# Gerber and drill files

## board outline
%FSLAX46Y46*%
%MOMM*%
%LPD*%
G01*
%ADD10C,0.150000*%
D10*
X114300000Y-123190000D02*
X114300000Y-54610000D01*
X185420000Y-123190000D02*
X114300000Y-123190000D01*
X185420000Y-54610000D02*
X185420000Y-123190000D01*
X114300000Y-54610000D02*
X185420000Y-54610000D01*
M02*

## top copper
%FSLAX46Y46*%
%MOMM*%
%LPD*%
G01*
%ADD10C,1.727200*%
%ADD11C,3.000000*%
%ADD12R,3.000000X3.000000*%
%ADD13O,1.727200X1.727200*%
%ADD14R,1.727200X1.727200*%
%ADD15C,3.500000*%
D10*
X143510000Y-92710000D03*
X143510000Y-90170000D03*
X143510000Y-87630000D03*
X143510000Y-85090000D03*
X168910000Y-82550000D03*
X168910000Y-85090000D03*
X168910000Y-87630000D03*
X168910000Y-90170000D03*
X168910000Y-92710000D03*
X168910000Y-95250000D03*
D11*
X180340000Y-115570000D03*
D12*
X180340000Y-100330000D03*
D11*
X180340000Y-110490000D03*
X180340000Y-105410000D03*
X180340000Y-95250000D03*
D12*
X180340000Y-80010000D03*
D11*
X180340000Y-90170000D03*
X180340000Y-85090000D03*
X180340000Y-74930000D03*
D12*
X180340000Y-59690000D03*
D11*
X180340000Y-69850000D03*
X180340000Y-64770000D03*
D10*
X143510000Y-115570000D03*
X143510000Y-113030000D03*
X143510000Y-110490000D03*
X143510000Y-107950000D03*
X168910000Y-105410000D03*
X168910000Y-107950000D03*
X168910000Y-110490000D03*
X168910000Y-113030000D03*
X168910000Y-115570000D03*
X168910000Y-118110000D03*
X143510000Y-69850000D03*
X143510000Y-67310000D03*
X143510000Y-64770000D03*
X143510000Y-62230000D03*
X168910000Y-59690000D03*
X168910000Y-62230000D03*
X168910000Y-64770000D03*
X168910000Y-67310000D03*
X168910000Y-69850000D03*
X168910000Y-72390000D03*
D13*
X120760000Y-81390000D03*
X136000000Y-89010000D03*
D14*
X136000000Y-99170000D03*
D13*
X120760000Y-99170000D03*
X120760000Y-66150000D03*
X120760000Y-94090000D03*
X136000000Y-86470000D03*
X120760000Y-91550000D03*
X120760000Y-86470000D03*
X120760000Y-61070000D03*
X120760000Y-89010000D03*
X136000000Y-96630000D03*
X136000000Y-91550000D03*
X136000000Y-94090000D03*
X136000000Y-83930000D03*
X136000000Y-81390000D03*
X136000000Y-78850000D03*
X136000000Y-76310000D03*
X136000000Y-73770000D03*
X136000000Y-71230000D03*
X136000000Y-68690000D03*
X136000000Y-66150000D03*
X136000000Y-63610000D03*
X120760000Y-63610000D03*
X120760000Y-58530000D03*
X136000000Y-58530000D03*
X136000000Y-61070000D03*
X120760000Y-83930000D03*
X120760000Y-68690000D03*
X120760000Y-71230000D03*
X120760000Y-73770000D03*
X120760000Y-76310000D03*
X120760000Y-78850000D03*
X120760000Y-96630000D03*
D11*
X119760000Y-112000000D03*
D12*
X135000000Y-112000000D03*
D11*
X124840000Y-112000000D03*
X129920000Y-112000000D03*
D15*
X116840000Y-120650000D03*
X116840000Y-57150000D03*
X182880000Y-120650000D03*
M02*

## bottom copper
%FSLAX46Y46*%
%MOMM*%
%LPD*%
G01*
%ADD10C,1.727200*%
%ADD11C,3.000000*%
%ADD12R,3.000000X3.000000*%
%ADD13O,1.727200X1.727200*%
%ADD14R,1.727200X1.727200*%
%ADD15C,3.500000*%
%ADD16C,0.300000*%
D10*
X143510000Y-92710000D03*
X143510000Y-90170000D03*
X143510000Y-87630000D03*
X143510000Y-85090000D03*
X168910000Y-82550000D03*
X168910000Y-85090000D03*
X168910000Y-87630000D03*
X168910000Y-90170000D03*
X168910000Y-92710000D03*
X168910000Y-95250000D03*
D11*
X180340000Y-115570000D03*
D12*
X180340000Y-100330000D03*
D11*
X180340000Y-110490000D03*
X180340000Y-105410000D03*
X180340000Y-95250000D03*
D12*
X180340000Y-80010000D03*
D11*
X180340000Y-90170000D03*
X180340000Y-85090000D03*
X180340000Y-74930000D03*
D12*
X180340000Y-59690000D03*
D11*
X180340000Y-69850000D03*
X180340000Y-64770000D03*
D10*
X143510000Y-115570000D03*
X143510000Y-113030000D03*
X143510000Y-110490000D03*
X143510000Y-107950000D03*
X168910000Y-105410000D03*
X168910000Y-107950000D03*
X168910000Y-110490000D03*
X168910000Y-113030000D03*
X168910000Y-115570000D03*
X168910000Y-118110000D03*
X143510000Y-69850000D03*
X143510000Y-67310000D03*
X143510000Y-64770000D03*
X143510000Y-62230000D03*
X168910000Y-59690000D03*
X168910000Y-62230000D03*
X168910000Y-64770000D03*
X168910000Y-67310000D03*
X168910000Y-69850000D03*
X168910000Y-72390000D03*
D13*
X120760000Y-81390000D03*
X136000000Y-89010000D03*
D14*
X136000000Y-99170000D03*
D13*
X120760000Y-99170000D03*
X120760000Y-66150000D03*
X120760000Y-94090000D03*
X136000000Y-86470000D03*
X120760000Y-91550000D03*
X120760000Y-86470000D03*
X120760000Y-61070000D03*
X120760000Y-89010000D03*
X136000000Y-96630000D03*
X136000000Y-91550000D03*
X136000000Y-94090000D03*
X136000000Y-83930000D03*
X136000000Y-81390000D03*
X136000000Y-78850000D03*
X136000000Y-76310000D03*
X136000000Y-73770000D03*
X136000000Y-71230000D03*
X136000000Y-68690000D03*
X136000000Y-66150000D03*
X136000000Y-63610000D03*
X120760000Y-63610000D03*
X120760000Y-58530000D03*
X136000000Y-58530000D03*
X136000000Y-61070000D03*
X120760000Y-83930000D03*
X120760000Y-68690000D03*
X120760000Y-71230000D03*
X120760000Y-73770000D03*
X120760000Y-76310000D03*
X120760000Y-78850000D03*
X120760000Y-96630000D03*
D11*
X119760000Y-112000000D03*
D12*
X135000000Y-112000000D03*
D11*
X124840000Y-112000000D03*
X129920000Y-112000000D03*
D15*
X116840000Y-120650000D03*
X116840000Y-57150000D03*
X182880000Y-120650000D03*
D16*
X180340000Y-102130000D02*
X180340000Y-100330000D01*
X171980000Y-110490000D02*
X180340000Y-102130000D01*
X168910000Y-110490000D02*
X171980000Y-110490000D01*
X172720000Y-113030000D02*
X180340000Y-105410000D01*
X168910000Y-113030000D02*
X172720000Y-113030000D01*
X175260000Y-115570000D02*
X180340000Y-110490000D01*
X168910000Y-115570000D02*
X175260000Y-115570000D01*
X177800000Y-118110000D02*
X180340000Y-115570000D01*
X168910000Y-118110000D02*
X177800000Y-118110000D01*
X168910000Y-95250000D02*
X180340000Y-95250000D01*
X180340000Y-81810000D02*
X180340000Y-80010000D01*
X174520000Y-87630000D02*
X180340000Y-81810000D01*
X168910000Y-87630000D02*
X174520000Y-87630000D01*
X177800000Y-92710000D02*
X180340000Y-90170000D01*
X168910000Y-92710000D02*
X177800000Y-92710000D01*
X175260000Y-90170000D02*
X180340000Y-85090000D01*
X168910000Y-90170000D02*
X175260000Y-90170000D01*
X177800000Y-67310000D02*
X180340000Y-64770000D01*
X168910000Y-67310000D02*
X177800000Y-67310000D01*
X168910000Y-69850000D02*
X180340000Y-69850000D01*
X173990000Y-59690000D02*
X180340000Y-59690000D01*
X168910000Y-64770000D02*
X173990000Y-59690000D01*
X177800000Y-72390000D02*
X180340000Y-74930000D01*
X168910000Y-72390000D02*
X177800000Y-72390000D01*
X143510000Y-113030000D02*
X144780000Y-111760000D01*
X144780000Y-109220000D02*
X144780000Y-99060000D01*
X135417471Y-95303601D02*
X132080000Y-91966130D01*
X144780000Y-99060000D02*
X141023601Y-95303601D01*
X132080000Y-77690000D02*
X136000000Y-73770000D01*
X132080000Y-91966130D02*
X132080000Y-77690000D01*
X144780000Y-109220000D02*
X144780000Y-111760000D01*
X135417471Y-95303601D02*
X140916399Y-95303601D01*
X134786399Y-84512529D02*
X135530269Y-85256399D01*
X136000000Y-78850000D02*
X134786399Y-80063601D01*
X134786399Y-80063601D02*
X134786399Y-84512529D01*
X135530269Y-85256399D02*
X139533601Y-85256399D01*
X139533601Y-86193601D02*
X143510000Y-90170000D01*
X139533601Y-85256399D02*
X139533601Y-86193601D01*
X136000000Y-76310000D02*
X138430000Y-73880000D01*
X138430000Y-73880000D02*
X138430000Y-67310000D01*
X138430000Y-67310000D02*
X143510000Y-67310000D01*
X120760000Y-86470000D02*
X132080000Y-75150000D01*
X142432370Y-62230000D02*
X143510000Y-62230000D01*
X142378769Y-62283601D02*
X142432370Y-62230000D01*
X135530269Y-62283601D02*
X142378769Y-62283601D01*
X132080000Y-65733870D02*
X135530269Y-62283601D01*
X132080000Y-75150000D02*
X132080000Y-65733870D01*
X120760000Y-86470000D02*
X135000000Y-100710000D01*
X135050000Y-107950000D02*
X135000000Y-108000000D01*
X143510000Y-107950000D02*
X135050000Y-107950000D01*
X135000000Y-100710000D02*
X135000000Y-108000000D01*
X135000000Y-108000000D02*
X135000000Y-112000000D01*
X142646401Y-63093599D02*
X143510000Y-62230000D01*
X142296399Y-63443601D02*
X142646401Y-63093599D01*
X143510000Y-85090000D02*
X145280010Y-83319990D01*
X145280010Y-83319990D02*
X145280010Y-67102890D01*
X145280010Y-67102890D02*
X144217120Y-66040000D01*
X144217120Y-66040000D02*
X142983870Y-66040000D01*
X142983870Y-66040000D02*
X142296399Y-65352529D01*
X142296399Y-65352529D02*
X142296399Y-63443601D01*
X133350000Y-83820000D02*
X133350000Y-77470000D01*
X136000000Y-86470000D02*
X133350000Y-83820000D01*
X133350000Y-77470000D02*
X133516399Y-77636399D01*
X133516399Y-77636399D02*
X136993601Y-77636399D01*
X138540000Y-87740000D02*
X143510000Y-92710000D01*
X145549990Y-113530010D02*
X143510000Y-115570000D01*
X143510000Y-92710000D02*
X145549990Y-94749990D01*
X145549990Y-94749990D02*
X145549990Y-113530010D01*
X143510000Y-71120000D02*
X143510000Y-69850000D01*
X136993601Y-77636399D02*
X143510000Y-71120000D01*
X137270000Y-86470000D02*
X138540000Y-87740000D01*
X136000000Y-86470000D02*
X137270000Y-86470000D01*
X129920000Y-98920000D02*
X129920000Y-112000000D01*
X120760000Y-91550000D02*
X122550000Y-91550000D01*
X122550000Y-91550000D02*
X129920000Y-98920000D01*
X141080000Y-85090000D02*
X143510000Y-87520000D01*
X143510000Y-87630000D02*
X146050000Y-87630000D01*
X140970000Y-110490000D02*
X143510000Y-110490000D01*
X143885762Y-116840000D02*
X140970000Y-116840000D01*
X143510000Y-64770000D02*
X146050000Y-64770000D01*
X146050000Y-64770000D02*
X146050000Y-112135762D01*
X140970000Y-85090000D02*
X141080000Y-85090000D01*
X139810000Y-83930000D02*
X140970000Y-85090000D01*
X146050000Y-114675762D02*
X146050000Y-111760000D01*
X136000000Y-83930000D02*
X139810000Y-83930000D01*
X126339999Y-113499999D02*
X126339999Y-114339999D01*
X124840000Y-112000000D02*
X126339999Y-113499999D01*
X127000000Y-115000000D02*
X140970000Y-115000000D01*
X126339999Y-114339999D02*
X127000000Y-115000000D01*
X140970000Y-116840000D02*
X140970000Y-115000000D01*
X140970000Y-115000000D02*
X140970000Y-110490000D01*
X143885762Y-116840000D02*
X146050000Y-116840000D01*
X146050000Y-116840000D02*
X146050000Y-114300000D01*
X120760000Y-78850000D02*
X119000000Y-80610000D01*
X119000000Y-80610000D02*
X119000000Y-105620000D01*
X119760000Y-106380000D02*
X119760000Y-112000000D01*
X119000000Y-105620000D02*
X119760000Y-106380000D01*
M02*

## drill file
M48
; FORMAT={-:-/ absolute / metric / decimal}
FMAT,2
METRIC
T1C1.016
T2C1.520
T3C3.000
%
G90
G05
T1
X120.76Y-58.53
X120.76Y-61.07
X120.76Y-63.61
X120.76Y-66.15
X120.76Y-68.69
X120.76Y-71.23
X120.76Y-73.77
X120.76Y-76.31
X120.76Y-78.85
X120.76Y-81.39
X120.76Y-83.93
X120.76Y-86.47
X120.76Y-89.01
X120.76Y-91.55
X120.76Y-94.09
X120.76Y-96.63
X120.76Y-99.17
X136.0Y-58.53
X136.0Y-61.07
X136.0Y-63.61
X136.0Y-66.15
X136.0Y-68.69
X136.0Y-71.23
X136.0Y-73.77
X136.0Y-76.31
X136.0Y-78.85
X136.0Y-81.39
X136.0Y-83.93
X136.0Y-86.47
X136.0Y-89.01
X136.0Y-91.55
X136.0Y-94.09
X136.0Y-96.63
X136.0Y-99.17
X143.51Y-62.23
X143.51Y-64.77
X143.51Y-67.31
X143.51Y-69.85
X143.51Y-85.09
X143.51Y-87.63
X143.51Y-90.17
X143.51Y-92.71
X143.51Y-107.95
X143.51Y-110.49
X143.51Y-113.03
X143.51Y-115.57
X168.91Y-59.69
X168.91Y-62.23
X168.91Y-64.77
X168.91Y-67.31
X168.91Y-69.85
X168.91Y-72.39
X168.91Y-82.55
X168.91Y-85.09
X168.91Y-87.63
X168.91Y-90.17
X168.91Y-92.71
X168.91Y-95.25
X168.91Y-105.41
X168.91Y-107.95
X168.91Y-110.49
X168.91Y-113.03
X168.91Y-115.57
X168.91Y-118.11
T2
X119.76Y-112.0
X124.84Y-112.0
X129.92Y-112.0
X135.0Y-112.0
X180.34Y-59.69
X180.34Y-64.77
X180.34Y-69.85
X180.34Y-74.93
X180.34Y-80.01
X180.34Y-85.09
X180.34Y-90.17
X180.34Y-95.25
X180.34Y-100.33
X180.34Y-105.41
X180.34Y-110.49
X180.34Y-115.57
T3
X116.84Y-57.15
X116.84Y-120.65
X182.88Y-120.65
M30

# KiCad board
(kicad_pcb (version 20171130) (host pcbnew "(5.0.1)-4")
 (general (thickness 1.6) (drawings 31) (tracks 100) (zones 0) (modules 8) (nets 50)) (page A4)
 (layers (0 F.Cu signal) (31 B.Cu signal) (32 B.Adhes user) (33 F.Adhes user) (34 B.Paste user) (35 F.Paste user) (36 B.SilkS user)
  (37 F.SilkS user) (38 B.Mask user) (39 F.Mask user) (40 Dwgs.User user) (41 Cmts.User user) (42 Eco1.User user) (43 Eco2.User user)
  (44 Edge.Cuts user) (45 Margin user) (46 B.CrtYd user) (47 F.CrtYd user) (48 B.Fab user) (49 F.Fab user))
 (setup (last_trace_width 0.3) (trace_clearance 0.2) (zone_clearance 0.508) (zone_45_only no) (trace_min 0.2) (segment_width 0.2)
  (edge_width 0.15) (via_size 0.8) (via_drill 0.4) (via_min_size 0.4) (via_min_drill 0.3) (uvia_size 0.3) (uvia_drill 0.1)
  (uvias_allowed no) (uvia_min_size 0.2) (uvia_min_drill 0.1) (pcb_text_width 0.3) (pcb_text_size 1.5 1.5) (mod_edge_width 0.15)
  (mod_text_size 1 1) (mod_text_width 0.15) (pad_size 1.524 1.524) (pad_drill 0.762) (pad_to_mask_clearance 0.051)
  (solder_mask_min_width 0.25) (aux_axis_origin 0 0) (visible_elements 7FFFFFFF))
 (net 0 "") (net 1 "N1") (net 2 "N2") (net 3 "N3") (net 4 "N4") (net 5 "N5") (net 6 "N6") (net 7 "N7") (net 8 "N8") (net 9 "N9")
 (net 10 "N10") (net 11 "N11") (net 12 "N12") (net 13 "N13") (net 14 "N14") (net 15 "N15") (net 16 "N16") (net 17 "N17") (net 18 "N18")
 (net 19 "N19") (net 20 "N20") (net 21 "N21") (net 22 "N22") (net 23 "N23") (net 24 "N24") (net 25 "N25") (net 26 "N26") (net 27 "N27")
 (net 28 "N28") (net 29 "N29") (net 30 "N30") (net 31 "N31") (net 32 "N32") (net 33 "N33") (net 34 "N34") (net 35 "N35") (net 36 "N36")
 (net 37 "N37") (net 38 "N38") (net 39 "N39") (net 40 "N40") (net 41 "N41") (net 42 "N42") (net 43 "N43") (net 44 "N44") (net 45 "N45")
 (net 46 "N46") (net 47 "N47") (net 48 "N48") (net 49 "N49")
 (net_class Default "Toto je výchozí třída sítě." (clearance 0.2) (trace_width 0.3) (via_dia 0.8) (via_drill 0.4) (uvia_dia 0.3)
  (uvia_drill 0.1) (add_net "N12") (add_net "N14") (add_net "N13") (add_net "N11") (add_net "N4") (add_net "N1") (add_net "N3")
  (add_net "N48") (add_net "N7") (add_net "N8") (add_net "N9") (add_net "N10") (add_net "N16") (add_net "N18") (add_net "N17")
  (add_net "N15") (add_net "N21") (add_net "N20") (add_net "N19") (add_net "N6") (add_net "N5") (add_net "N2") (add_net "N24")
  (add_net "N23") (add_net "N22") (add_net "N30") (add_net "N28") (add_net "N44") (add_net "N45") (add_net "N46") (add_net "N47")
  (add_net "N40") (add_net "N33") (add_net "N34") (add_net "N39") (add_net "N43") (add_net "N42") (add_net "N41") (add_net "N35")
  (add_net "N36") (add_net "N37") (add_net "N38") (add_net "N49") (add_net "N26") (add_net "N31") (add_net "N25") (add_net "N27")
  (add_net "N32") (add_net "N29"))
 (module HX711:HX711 (layer F.Cu) (at 167.64 91.44 180)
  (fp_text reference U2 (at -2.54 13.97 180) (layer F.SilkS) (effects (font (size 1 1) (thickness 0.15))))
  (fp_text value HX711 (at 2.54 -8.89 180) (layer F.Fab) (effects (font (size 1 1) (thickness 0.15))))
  (pad 7 thru_hole circle (at 24.13 -1.27 180) (size 1.7272 1.7272) (drill 1.016) (layers *.Cu *.Mask) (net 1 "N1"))
  (pad 8 thru_hole circle (at 24.13 1.27 180) (size 1.7272 1.7272) (drill 1.016) (layers *.Cu *.Mask) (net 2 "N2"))
  (pad 9 thru_hole circle (at 24.13 3.81 180) (size 1.7272 1.7272) (drill 1.016) (layers *.Cu *.Mask) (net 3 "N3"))
  (pad 10 thru_hole circle (at 24.13 6.35 180) (size 1.7272 1.7272) (drill 1.016) (layers *.Cu *.Mask) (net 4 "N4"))
  (pad 6 thru_hole circle (at -1.27 8.89 180) (size 1.7272 1.7272) (drill 1.016) (layers *.Cu *.Mask) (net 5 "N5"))
  (pad 5 thru_hole circle (at -1.27 6.35 180) (size 1.7272 1.7272) (drill 1.016) (layers *.Cu *.Mask) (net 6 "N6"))
  (pad 4 thru_hole circle (at -1.27 3.81 180) (size 1.7272 1.7272) (drill 1.016) (layers *.Cu *.Mask) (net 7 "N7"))
  (pad 3 thru_hole circle (at -1.27 1.27 180) (size 1.7272 1.7272) (drill 1.016) (layers *.Cu *.Mask) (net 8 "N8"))
  (pad 2 thru_hole circle (at -1.27 -1.27 180) (size 1.7272 1.7272) (drill 1.016) (layers *.Cu *.Mask) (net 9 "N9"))
  (pad 1 thru_hole circle (at -1.27 -3.81 180) (size 1.7272 1.7272) (drill 1.016) (layers *.Cu *.Mask) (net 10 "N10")))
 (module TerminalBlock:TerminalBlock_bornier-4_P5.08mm (layer F.Cu) (at 180.34 100.33 270)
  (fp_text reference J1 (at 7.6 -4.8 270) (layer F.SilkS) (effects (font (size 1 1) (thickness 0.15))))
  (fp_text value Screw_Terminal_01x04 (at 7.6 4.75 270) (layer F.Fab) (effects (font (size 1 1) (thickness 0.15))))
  (pad 4 thru_hole circle (at 15.24 0 270) (size 3 3) (drill 1.52) (layers *.Cu *.Mask) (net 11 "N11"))
  (pad 1 thru_hole rect (at 0 0 270) (size 3 3) (drill 1.52) (layers *.Cu *.Mask) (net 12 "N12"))
  (pad 3 thru_hole circle (at 10.16 0 270) (size 3 3) (drill 1.52) (layers *.Cu *.Mask) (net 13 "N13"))
  (pad 2 thru_hole circle (at 5.08 0 270) (size 3 3) (drill 1.52) (layers *.Cu *.Mask) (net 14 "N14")))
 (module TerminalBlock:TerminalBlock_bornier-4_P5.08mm (layer F.Cu) (at 180.34 80.01 270)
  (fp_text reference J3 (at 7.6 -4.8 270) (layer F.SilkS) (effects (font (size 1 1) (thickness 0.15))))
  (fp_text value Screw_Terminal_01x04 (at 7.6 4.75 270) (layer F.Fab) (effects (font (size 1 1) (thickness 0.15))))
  (pad 4 thru_hole circle (at 15.24 0 270) (size 3 3) (drill 1.52) (layers *.Cu *.Mask) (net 10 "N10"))
  (pad 1 thru_hole rect (at 0 0 270) (size 3 3) (drill 1.52) (layers *.Cu *.Mask) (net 7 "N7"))
  (pad 3 thru_hole circle (at 10.16 0 270) (size 3 3) (drill 1.52) (layers *.Cu *.Mask) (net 9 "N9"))
  (pad 2 thru_hole circle (at 5.08 0 270) (size 3 3) (drill 1.52) (layers *.Cu *.Mask) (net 8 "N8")))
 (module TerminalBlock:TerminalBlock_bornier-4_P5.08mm (layer F.Cu) (at 180.34 59.69 270)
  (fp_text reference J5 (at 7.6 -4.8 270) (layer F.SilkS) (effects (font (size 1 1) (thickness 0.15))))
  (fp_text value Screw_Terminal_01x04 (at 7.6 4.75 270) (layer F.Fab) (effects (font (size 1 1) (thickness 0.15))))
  (pad 4 thru_hole circle (at 15.24 0 270) (size 3 3) (drill 1.52) (layers *.Cu *.Mask) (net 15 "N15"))
  (pad 1 thru_hole rect (at 0 0 270) (size 3 3) (drill 1.52) (layers *.Cu *.Mask) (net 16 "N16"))
  (pad 3 thru_hole circle (at 10.16 0 270) (size 3 3) (drill 1.52) (layers *.Cu *.Mask) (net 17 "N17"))
  (pad 2 thru_hole circle (at 5.08 0 270) (size 3 3) (drill 1.52) (layers *.Cu *.Mask) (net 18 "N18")))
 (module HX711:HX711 (layer F.Cu) (at 167.64 114.3 180)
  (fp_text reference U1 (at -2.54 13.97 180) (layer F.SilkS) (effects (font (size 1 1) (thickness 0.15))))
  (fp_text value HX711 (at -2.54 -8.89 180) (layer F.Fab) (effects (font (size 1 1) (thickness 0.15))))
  (pad 7 thru_hole circle (at 24.13 -1.27 180) (size 1.7272 1.7272) (drill 1.016) (layers *.Cu *.Mask) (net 1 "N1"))
  (pad 8 thru_hole circle (at 24.13 1.27 180) (size 1.7272 1.7272) (drill 1.016) (layers *.Cu *.Mask) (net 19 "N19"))
  (pad 9 thru_hole circle (at 24.13 3.81 180) (size 1.7272 1.7272) (drill 1.016) (layers *.Cu *.Mask) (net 3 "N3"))
  (pad 10 thru_hole circle (at 24.13 6.35 180) (size 1.7272 1.7272) (drill 1.016) (layers *.Cu *.Mask) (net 4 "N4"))
  (pad 6 thru_hole circle (at -1.27 8.89 180) (size 1.7272 1.7272) (drill 1.016) (layers *.Cu *.Mask) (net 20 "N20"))
  (pad 5 thru_hole circle (at -1.27 6.35 180) (size 1.7272 1.7272) (drill 1.016) (layers *.Cu *.Mask) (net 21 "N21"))
  (pad 4 thru_hole circle (at -1.27 3.81 180) (size 1.7272 1.7272) (drill 1.016) (layers *.Cu *.Mask) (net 12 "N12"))
  (pad 3 thru_hole circle (at -1.27 1.27 180) (size 1.7272 1.7272) (drill 1.016) (layers *.Cu *.Mask) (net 14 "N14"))
  (pad 2 thru_hole circle (at -1.27 -1.27 180) (size 1.7272 1.7272) (drill 1.016) (layers *.Cu *.Mask) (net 13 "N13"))
  (pad 1 thru_hole circle (at -1.27 -3.81 180) (size 1.7272 1.7272) (drill 1.016) (layers *.Cu *.Mask) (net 11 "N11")))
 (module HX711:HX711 (layer F.Cu) (at 167.64 68.58 180)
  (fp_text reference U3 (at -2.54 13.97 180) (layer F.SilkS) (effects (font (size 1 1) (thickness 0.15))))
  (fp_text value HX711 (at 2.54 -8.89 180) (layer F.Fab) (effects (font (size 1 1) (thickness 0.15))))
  (pad 7 thru_hole circle (at 24.13 -1.27 180) (size 1.7272 1.7272) (drill 1.016) (layers *.Cu *.Mask) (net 1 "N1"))
  (pad 8 thru_hole circle (at 24.13 1.27 180) (size 1.7272 1.7272) (drill 1.016) (layers *.Cu *.Mask) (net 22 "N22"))
  (pad 9 thru_hole circle (at 24.13 3.81 180) (size 1.7272 1.7272) (drill 1.016) (layers *.Cu *.Mask) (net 3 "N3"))
  (pad 10 thru_hole circle (at 24.13 6.35 180) (size 1.7272 1.7272) (drill 1.016) (layers *.Cu *.Mask) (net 4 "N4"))
  (pad 6 thru_hole circle (at -1.27 8.89 180) (size 1.7272 1.7272) (drill 1.016) (layers *.Cu *.Mask) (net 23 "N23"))
  (pad 5 thru_hole circle (at -1.27 6.35 180) (size 1.7272 1.7272) (drill 1.016) (layers *.Cu *.Mask) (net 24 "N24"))
  (pad 4 thru_hole circle (at -1.27 3.81 180) (size 1.7272 1.7272) (drill 1.016) (layers *.Cu *.Mask) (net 16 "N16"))
  (pad 3 thru_hole circle (at -1.27 1.27 180) (size 1.7272 1.7272) (drill 1.016) (layers *.Cu *.Mask) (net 18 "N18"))
  (pad 2 thru_hole circle (at -1.27 -1.27 180) (size 1.7272 1.7272) (drill 1.016) (layers *.Cu *.Mask) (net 17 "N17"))
  (pad 1 thru_hole circle (at -1.27 -3.81 180) (size 1.7272 1.7272) (drill 1.016) (layers *.Cu *.Mask) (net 15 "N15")))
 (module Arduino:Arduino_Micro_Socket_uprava (layer F.Cu) (at 119.38 54.61 270)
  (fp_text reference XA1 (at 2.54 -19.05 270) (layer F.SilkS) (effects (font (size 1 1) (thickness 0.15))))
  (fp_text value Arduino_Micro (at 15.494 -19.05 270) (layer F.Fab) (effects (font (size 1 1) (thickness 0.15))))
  (pad "" thru_hole oval (at 26.78 -1.38 270) (size 1.7272 1.7272) (drill 1.016) (layers *.Cu *.Mask))
  (pad RST2 thru_hole oval (at 34.4 -16.62 270) (size 1.7272 1.7272) (drill 1.016) (layers *.Cu *.Mask) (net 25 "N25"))
  (pad MOSI thru_hole rect (at 44.56 -16.62 270) (size 1.7272 1.7272) (drill 1.016) (layers *.Cu *.Mask) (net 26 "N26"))
  (pad SCK thru_hole oval (at 44.56 -1.38 270) (size 1.7272 1.7272) (drill 1.016) (layers *.Cu *.Mask) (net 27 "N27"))
  (pad A0 thru_hole oval (at 11.54 -1.38 270) (size 1.7272 1.7272) (drill 1.016) (layers *.Cu *.Mask) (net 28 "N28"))
  (pad VIN thru_hole oval (at 39.48 -1.38 270) (size 1.7272 1.7272) (drill 1.016) (layers *.Cu *.Mask) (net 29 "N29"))
  (pad GND2 thru_hole oval (at 31.86 -16.62 270) (size 1.7272 1.7272) (drill 1.016) (layers *.Cu *.Mask) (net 1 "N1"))
  (pad GND1 thru_hole oval (at 36.94 -1.38 270) (size 1.7272 1.7272) (drill 1.016) (layers *.Cu *.Mask) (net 1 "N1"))
  (pad 5V thru_hole oval (at 31.86 -1.38 270) (size 1.7272 1.7272) (drill 1.016) (layers *.Cu *.Mask) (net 4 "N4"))
  (pad 3V3 thru_hole oval (at 6.46 -1.38 270) (size 1.7272 1.7272) (drill 1.016) (layers *.Cu *.Mask) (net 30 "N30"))
  (pad RST1 thru_hole oval (at 34.4 -1.38 270) (size 1.7272 1.7272) (drill 1.016) (layers *.Cu *.Mask) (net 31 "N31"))
  (pad SS thru_hole oval (at 42.02 -16.62 270) (size 1.7272 1.7272) (drill 1.016) (layers *.Cu *.Mask) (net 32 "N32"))
  (pad D0 thru_hole oval (at 36.94 -16.62 270) (size 1.7272 1.7272) (drill 1.016) (layers *.Cu *.Mask) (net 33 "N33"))
  (pad D1 thru_hole oval (at 39.48 -16.62 270) (size 1.7272 1.7272) (drill 1.016) (layers *.Cu *.Mask) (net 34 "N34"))
  (pad D2 thru_hole oval (at 29.32 -16.62 270) (size 1.7272 1.7272) (drill 1.016) (layers *.Cu *.Mask) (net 3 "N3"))
  (pad D3 thru_hole oval (at 26.78 -16.62 270) (size 1.7272 1.7272) (drill 1.016) (layers *.Cu *.Mask) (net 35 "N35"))
  (pad D4 thru_hole oval (at 24.24 -16.62 270) (size 1.7272 1.7272) (drill 1.016) (layers *.Cu *.Mask) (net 2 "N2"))
  (pad D5 thru_hole oval (at 21.7 -16.62 270) (size 1.7272 1.7272) (drill 1.016) (layers *.Cu *.Mask) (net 22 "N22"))
  (pad D6 thru_hole oval (at 19.16 -16.62 270) (size 1.7272 1.7272) (drill 1.016) (layers *.Cu *.Mask) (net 19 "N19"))
  (pad D7 thru_hole oval (at 16.62 -16.62 270) (size 1.7272 1.7272) (drill 1.016) (layers *.Cu *.Mask) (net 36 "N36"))
  (pad D8 thru_hole oval (at 14.08 -16.62 270) (size 1.7272 1.7272) (drill 1.016) (layers *.Cu *.Mask) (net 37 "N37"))
  (pad D9 thru_hole oval (at 11.54 -16.62 270) (size 1.7272 1.7272) (drill 1.016) (layers *.Cu *.Mask) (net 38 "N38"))
  (pad D10 thru_hole oval (at 9 -16.62 270) (size 1.7272 1.7272) (drill 1.016) (layers *.Cu *.Mask) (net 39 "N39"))
  (pad AREF thru_hole oval (at 9 -1.38 270) (size 1.7272 1.7272) (drill 1.016) (layers *.Cu *.Mask) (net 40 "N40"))
  (pad D13 thru_hole oval (at 3.92 -1.38 270) (size 1.7272 1.7272) (drill 1.016) (layers *.Cu *.Mask) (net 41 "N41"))
  (pad D12 thru_hole oval (at 3.92 -16.62 270) (size 1.7272 1.7272) (drill 1.016) (layers *.Cu *.Mask) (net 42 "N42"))
  (pad D11 thru_hole oval (at 6.46 -16.62 270) (size 1.7272 1.7272) (drill 1.016) (layers *.Cu *.Mask) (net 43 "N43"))
  (pad "" thru_hole oval (at 29.32 -1.38 270) (size 1.7272 1.7272) (drill 1.016) (layers *.Cu *.Mask))
  (pad A1 thru_hole oval (at 14.08 -1.38 270) (size 1.7272 1.7272) (drill 1.016) (layers *.Cu *.Mask) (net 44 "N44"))
  (pad A2 thru_hole oval (at 16.62 -1.38 270) (size 1.7272 1.7272) (drill 1.016) (layers *.Cu *.Mask) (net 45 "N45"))
  (pad A3 thru_hole oval (at 19.16 -1.38 270) (size 1.7272 1.7272) (drill 1.016) (layers *.Cu *.Mask) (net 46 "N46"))
  (pad A4 thru_hole oval (at 21.7 -1.38 270) (size 1.7272 1.7272) (drill 1.016) (layers *.Cu *.Mask) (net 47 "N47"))
  (pad A5 thru_hole oval (at 24.24 -1.38 270) (size 1.7272 1.7272) (drill 1.016) (layers *.Cu *.Mask) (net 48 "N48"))
  (pad MISO thru_hole oval (at 42.02 -1.38 270) (size 1.7272 1.7272) (drill 1.016) (layers *.Cu *.Mask) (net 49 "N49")))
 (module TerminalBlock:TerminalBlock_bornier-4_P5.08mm (layer F.Cu) (at 135 112 180)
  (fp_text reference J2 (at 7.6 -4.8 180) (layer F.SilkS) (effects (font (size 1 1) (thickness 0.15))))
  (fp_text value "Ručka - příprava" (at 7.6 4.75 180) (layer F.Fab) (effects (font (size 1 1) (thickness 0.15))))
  (pad 4 thru_hole circle (at 15.24 0 180) (size 3 3) (drill 1.52) (layers *.Cu *.Mask) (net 48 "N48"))
  (pad 1 thru_hole rect (at 0 0 180) (size 3 3) (drill 1.52) (layers *.Cu *.Mask) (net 4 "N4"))
  (pad 3 thru_hole circle (at 10.16 0 180) (size 3 3) (drill 1.52) (layers *.Cu *.Mask) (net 3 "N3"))
  (pad 2 thru_hole circle (at 5.08 0 180) (size 3 3) (drill 1.52) (layers *.Cu *.Mask) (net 1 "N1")))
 (gr_line (start 114.3 123.19) (end 114.3 54.61) (layer Edge.Cuts) (width 0.15))
 (gr_line (start 185.42 123.19) (end 114.3 123.19) (layer Edge.Cuts) (width 0.15))
 (gr_line (start 185.42 54.61) (end 185.42 123.19) (layer Edge.Cuts) (width 0.15))
 (gr_line (start 114.3 54.61) (end 185.42 54.61) (layer Edge.Cuts) (width 0.15))
 (via (at 116.84 120.65) (size 3.5) (drill 3) (layers F.Cu B.Cu) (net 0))
 (via (at 116.84 57.15) (size 3.5) (drill 3) (layers F.Cu B.Cu) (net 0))
 (via (at 182.88 120.65) (size 3.5) (drill 3) (layers F.Cu B.Cu) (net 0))
 (segment (start 180.34 102.13) (end 180.34 100.33) (width 0.3) (layer B.Cu) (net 12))
 (segment (start 171.98 110.49) (end 180.34 102.13) (width 0.3) (layer B.Cu) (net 12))
 (segment (start 168.91 110.49) (end 171.98 110.49) (width 0.3) (layer B.Cu) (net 12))
 (segment (start 172.72 113.03) (end 180.34 105.41) (width 0.3) (layer B.Cu) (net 14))
 (segment (start 168.91 113.03) (end 172.72 113.03) (width 0.3) (layer B.Cu) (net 14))
 (segment (start 175.26 115.57) (end 180.34 110.49) (width 0.3) (layer B.Cu) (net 13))
 (segment (start 168.91 115.57) (end 175.26 115.57) (width 0.3) (layer B.Cu) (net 13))
 (segment (start 177.8 118.11) (end 180.34 115.57) (width 0.3) (layer B.Cu) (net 11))
 (segment (start 168.91 118.11) (end 177.8 118.11) (width 0.3) (layer B.Cu) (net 11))
 (segment (start 168.91 95.25) (end 180.34 95.25) (width 0.3) (layer B.Cu) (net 10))
 (segment (start 180.34 81.81) (end 180.34 80.01) (width 0.3) (layer B.Cu) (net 7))
 (segment (start 174.52 87.63) (end 180.34 81.81) (width 0.3) (layer B.Cu) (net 7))
 (segment (start 168.91 87.63) (end 174.52 87.63) (width 0.3) (layer B.Cu) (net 7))
 (segment (start 177.8 92.71) (end 180.34 90.17) (width 0.3) (layer B.Cu) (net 9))
 (segment (start 168.91 92.71) (end 177.8 92.71) (width 0.3) (layer B.Cu) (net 9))
 (segment (start 175.26 90.17) (end 180.34 85.09) (width 0.3) (layer B.Cu) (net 8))
 (segment (start 168.91 90.17) (end 175.26 90.17) (width 0.3) (layer B.Cu) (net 8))
 (segment (start 177.8 67.31) (end 180.34 64.77) (width 0.3) (layer B.Cu) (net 18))
 (segment (start 168.91 67.31) (end 177.8 67.31) (width 0.3) (layer B.Cu) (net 18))
 (segment (start 168.91 69.85) (end 180.34 69.85) (width 0.3) (layer B.Cu) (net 17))
 (segment (start 173.99 59.69) (end 180.34 59.69) (width 0.3) (layer B.Cu) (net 16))
 (segment (start 168.91 64.77) (end 173.99 59.69) (width 0.3) (layer B.Cu) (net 16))
 (segment (start 177.8 72.39) (end 180.34 74.93) (width 0.3) (layer B.Cu) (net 15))
 (segment (start 168.91 72.39) (end 177.8 72.39) (width 0.3) (layer B.Cu) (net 15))
 (segment (start 143.51 113.03) (end 144.78 111.76) (width 0.3) (layer B.Cu) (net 19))
 (segment (start 144.78 109.22) (end 144.78 99.06) (width 0.3) (layer B.Cu) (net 19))
 (segment (start 135.417471 95.303601) (end 132.08 91.96613) (width 0.3) (layer B.Cu) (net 19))
 (segment (start 144.78 99.06) (end 141.023601 95.303601) (width 0.3) (layer B.Cu) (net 19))
 (segment (start 132.08 77.69) (end 136 73.77) (width 0.3) (layer B.Cu) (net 19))
 (segment (start 132.08 91.96613) (end 132.08 77.69) (width 0.3) (layer B.Cu) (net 19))
 (segment (start 144.78 109.22) (end 144.78 111.76) (width 0.3) (layer B.Cu) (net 19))
 (segment (start 135.417471 95.303601) (end 140.916399 95.303601) (width 0.3) (layer B.Cu) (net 19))
 (segment (start 134.786399 84.512529) (end 135.530269 85.256399) (width 0.3) (layer B.Cu) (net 2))
 (segment (start 136 78.85) (end 134.786399 80.063601) (width 0.3) (layer B.Cu) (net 2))
 (segment (start 134.786399 80.063601) (end 134.786399 84.512529) (width 0.3) (layer B.Cu) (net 2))
 (segment (start 135.530269 85.256399) (end 139.533601 85.256399) (width 0.3) (layer B.Cu) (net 2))
 (segment (start 139.533601 86.193601) (end 143.51 90.17) (width 0.3) (layer B.Cu) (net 2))
 (segment (start 139.533601 85.256399) (end 139.533601 86.193601) (width 0.3) (layer B.Cu) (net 2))
 (segment (start 136 76.31) (end 138.43 73.88) (width 0.3) (layer B.Cu) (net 22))
 (segment (start 138.43 73.88) (end 138.43 67.31) (width 0.3) (layer B.Cu) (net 22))
 (segment (start 138.43 67.31) (end 143.51 67.31) (width 0.3) (layer B.Cu) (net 22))
 (segment (start 120.76 86.47) (end 132.08 75.15) (width 0.3) (layer B.Cu) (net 4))
 (segment (start 142.43237 62.23) (end 143.51 62.23) (width 0.3) (layer B.Cu) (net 4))
 (segment (start 142.378769 62.283601) (end 142.43237 62.23) (width 0.3) (layer B.Cu) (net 4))
 (segment (start 135.530269 62.283601) (end 142.378769 62.283601) (width 0.3) (layer B.Cu) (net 4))
 (segment (start 132.08 65.73387) (end 135.530269 62.283601) (width 0.3) (layer B.Cu) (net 4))
 (segment (start 132.08 75.15) (end 132.08 65.73387) (width 0.3) (layer B.Cu) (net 4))
 (segment (start 120.76 86.47) (end 135 100.71) (width 0.3) (layer B.Cu) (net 4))
 (segment (start 135.05 107.95) (end 135 108) (width 0.3) (layer B.Cu) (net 4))
 (segment (start 143.51 107.95) (end 135.05 107.95) (width 0.3) (layer B.Cu) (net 4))
 (segment (start 135 100.71) (end 135 108) (width 0.3) (layer B.Cu) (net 4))
 (segment (start 135 108) (end 135 112) (width 0.3) (layer B.Cu) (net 4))
 (segment (start 142.646401 63.093599) (end 143.51 62.23) (width 0.3) (layer B.Cu) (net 4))
 (segment (start 142.296399 63.443601) (end 142.646401 63.093599) (width 0.3) (layer B.Cu) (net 4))
 (segment (start 143.51 85.09) (end 145.28001 83.31999) (width 0.3) (layer B.Cu) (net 4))
 (segment (start 145.28001 83.31999) (end 145.28001 67.10289) (width 0.3) (layer B.Cu) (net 4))
 (segment (start 145.28001 67.10289) (end 144.21712 66.04) (width 0.3) (layer B.Cu) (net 4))
 (segment (start 144.21712 66.04) (end 142.98387 66.04) (width 0.3) (layer B.Cu) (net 4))
 (segment (start 142.98387 66.04) (end 142.296399 65.352529) (width 0.3) (layer B.Cu) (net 4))
 (segment (start 142.296399 65.352529) (end 142.296399 63.443601) (width 0.3) (layer B.Cu) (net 4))
 (segment (start 133.35 83.82) (end 133.35 77.47) (width 0.3) (layer B.Cu) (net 1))
 (segment (start 136 86.47) (end 133.35 83.82) (width 0.3) (layer B.Cu) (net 1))
 (segment (start 133.35 77.47) (end 133.516399 77.636399) (width 0.3) (layer B.Cu) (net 1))
 (segment (start 133.516399 77.636399) (end 136.993601 77.636399) (width 0.3) (layer B.Cu) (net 1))
 (segment (start 138.54 87.74) (end 143.51 92.71) (width 0.3) (layer B.Cu) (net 1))
 (segment (start 145.54999 113.53001) (end 143.51 115.57) (width 0.3) (layer B.Cu) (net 1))
 (segment (start 143.51 92.71) (end 145.54999 94.74999) (width 0.3) (layer B.Cu) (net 1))
 (segment (start 145.54999 94.74999) (end 145.54999 113.53001) (width 0.3) (layer B.Cu) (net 1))
 (segment (start 143.51 71.12) (end 143.51 69.85) (width 0.3) (layer B.Cu) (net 1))
 (segment (start 136.993601 77.636399) (end 143.51 71.12) (width 0.3) (layer B.Cu) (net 1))
 (segment (start 137.27 86.47) (end 138.54 87.74) (width 0.3) (layer B.Cu) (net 1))
 (segment (start 136 86.47) (end 137.27 86.47) (width 0.3) (layer B.Cu) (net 1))
 (segment (start 129.92 98.92) (end 129.92 112) (width 0.3) (layer B.Cu) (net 1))
 (segment (start 120.76 91.55) (end 122.55 91.55) (width 0.3) (layer B.Cu) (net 1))
 (segment (start 122.55 91.55) (end 129.92 98.92) (width 0.3) (layer B.Cu) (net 1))
 (segment (start 141.08 85.09) (end 143.51 87.52) (width 0.3) (layer B.Cu) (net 3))
 (segment (start 143.51 87.63) (end 146.05 87.63) (width 0.3) (layer B.Cu) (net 3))
 (segment (start 140.97 110.49) (end 143.51 110.49) (width 0.3) (layer B.Cu) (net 3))
 (segment (start 143.885762 116.84) (end 140.97 116.84) (width 0.3) (layer B.Cu) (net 3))
 (segment (start 143.51 64.77) (end 146.05 64.77) (width 0.3) (layer B.Cu) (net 3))
 (segment (start 146.05 64.77) (end 146.05 112.135762) (width 0.3) (layer B.Cu) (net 3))
 (segment (start 140.97 85.09) (end 141.08 85.09) (width 0.3) (layer B.Cu) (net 3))
 (segment (start 139.81 83.93) (end 140.97 85.09) (width 0.3) (layer B.Cu) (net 3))
 (segment (start 146.05 114.675762) (end 146.05 111.76) (width 0.3) (layer B.Cu) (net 3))
 (segment (start 136 83.93) (end 139.81 83.93) (width 0.3) (layer B.Cu) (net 3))
 (segment (start 126.339999 113.499999) (end 126.339999 114.339999) (width 0.3) (layer B.Cu) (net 3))
 (segment (start 124.84 112) (end 126.339999 113.499999) (width 0.3) (layer B.Cu) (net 3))
 (segment (start 127 115) (end 140.97 115) (width 0.3) (layer B.Cu) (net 3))
 (segment (start 126.339999 114.339999) (end 127 115) (width 0.3) (layer B.Cu) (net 3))
 (segment (start 140.97 116.84) (end 140.97 115) (width 0.3) (layer B.Cu) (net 3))
 (segment (start 140.97 115) (end 140.97 110.49) (width 0.3) (layer B.Cu) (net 3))
 (segment (start 143.885762 116.84) (end 146.05 116.84) (width 0.3) (layer B.Cu) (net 3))
 (segment (start 146.05 116.84) (end 146.05 114.3) (width 0.3) (layer B.Cu) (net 3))
 (segment (start 120.76 78.85) (end 119 80.61) (width 0.3) (layer B.Cu) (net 48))
 (segment (start 119 80.61) (end 119 105.62) (width 0.3) (layer B.Cu) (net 48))
 (segment (start 119.76 106.38) (end 119.76 112) (width 0.3) (layer B.Cu) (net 48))
 (segment (start 119 105.62) (end 119.76 106.38) (width 0.3) (layer B.Cu) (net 48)))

